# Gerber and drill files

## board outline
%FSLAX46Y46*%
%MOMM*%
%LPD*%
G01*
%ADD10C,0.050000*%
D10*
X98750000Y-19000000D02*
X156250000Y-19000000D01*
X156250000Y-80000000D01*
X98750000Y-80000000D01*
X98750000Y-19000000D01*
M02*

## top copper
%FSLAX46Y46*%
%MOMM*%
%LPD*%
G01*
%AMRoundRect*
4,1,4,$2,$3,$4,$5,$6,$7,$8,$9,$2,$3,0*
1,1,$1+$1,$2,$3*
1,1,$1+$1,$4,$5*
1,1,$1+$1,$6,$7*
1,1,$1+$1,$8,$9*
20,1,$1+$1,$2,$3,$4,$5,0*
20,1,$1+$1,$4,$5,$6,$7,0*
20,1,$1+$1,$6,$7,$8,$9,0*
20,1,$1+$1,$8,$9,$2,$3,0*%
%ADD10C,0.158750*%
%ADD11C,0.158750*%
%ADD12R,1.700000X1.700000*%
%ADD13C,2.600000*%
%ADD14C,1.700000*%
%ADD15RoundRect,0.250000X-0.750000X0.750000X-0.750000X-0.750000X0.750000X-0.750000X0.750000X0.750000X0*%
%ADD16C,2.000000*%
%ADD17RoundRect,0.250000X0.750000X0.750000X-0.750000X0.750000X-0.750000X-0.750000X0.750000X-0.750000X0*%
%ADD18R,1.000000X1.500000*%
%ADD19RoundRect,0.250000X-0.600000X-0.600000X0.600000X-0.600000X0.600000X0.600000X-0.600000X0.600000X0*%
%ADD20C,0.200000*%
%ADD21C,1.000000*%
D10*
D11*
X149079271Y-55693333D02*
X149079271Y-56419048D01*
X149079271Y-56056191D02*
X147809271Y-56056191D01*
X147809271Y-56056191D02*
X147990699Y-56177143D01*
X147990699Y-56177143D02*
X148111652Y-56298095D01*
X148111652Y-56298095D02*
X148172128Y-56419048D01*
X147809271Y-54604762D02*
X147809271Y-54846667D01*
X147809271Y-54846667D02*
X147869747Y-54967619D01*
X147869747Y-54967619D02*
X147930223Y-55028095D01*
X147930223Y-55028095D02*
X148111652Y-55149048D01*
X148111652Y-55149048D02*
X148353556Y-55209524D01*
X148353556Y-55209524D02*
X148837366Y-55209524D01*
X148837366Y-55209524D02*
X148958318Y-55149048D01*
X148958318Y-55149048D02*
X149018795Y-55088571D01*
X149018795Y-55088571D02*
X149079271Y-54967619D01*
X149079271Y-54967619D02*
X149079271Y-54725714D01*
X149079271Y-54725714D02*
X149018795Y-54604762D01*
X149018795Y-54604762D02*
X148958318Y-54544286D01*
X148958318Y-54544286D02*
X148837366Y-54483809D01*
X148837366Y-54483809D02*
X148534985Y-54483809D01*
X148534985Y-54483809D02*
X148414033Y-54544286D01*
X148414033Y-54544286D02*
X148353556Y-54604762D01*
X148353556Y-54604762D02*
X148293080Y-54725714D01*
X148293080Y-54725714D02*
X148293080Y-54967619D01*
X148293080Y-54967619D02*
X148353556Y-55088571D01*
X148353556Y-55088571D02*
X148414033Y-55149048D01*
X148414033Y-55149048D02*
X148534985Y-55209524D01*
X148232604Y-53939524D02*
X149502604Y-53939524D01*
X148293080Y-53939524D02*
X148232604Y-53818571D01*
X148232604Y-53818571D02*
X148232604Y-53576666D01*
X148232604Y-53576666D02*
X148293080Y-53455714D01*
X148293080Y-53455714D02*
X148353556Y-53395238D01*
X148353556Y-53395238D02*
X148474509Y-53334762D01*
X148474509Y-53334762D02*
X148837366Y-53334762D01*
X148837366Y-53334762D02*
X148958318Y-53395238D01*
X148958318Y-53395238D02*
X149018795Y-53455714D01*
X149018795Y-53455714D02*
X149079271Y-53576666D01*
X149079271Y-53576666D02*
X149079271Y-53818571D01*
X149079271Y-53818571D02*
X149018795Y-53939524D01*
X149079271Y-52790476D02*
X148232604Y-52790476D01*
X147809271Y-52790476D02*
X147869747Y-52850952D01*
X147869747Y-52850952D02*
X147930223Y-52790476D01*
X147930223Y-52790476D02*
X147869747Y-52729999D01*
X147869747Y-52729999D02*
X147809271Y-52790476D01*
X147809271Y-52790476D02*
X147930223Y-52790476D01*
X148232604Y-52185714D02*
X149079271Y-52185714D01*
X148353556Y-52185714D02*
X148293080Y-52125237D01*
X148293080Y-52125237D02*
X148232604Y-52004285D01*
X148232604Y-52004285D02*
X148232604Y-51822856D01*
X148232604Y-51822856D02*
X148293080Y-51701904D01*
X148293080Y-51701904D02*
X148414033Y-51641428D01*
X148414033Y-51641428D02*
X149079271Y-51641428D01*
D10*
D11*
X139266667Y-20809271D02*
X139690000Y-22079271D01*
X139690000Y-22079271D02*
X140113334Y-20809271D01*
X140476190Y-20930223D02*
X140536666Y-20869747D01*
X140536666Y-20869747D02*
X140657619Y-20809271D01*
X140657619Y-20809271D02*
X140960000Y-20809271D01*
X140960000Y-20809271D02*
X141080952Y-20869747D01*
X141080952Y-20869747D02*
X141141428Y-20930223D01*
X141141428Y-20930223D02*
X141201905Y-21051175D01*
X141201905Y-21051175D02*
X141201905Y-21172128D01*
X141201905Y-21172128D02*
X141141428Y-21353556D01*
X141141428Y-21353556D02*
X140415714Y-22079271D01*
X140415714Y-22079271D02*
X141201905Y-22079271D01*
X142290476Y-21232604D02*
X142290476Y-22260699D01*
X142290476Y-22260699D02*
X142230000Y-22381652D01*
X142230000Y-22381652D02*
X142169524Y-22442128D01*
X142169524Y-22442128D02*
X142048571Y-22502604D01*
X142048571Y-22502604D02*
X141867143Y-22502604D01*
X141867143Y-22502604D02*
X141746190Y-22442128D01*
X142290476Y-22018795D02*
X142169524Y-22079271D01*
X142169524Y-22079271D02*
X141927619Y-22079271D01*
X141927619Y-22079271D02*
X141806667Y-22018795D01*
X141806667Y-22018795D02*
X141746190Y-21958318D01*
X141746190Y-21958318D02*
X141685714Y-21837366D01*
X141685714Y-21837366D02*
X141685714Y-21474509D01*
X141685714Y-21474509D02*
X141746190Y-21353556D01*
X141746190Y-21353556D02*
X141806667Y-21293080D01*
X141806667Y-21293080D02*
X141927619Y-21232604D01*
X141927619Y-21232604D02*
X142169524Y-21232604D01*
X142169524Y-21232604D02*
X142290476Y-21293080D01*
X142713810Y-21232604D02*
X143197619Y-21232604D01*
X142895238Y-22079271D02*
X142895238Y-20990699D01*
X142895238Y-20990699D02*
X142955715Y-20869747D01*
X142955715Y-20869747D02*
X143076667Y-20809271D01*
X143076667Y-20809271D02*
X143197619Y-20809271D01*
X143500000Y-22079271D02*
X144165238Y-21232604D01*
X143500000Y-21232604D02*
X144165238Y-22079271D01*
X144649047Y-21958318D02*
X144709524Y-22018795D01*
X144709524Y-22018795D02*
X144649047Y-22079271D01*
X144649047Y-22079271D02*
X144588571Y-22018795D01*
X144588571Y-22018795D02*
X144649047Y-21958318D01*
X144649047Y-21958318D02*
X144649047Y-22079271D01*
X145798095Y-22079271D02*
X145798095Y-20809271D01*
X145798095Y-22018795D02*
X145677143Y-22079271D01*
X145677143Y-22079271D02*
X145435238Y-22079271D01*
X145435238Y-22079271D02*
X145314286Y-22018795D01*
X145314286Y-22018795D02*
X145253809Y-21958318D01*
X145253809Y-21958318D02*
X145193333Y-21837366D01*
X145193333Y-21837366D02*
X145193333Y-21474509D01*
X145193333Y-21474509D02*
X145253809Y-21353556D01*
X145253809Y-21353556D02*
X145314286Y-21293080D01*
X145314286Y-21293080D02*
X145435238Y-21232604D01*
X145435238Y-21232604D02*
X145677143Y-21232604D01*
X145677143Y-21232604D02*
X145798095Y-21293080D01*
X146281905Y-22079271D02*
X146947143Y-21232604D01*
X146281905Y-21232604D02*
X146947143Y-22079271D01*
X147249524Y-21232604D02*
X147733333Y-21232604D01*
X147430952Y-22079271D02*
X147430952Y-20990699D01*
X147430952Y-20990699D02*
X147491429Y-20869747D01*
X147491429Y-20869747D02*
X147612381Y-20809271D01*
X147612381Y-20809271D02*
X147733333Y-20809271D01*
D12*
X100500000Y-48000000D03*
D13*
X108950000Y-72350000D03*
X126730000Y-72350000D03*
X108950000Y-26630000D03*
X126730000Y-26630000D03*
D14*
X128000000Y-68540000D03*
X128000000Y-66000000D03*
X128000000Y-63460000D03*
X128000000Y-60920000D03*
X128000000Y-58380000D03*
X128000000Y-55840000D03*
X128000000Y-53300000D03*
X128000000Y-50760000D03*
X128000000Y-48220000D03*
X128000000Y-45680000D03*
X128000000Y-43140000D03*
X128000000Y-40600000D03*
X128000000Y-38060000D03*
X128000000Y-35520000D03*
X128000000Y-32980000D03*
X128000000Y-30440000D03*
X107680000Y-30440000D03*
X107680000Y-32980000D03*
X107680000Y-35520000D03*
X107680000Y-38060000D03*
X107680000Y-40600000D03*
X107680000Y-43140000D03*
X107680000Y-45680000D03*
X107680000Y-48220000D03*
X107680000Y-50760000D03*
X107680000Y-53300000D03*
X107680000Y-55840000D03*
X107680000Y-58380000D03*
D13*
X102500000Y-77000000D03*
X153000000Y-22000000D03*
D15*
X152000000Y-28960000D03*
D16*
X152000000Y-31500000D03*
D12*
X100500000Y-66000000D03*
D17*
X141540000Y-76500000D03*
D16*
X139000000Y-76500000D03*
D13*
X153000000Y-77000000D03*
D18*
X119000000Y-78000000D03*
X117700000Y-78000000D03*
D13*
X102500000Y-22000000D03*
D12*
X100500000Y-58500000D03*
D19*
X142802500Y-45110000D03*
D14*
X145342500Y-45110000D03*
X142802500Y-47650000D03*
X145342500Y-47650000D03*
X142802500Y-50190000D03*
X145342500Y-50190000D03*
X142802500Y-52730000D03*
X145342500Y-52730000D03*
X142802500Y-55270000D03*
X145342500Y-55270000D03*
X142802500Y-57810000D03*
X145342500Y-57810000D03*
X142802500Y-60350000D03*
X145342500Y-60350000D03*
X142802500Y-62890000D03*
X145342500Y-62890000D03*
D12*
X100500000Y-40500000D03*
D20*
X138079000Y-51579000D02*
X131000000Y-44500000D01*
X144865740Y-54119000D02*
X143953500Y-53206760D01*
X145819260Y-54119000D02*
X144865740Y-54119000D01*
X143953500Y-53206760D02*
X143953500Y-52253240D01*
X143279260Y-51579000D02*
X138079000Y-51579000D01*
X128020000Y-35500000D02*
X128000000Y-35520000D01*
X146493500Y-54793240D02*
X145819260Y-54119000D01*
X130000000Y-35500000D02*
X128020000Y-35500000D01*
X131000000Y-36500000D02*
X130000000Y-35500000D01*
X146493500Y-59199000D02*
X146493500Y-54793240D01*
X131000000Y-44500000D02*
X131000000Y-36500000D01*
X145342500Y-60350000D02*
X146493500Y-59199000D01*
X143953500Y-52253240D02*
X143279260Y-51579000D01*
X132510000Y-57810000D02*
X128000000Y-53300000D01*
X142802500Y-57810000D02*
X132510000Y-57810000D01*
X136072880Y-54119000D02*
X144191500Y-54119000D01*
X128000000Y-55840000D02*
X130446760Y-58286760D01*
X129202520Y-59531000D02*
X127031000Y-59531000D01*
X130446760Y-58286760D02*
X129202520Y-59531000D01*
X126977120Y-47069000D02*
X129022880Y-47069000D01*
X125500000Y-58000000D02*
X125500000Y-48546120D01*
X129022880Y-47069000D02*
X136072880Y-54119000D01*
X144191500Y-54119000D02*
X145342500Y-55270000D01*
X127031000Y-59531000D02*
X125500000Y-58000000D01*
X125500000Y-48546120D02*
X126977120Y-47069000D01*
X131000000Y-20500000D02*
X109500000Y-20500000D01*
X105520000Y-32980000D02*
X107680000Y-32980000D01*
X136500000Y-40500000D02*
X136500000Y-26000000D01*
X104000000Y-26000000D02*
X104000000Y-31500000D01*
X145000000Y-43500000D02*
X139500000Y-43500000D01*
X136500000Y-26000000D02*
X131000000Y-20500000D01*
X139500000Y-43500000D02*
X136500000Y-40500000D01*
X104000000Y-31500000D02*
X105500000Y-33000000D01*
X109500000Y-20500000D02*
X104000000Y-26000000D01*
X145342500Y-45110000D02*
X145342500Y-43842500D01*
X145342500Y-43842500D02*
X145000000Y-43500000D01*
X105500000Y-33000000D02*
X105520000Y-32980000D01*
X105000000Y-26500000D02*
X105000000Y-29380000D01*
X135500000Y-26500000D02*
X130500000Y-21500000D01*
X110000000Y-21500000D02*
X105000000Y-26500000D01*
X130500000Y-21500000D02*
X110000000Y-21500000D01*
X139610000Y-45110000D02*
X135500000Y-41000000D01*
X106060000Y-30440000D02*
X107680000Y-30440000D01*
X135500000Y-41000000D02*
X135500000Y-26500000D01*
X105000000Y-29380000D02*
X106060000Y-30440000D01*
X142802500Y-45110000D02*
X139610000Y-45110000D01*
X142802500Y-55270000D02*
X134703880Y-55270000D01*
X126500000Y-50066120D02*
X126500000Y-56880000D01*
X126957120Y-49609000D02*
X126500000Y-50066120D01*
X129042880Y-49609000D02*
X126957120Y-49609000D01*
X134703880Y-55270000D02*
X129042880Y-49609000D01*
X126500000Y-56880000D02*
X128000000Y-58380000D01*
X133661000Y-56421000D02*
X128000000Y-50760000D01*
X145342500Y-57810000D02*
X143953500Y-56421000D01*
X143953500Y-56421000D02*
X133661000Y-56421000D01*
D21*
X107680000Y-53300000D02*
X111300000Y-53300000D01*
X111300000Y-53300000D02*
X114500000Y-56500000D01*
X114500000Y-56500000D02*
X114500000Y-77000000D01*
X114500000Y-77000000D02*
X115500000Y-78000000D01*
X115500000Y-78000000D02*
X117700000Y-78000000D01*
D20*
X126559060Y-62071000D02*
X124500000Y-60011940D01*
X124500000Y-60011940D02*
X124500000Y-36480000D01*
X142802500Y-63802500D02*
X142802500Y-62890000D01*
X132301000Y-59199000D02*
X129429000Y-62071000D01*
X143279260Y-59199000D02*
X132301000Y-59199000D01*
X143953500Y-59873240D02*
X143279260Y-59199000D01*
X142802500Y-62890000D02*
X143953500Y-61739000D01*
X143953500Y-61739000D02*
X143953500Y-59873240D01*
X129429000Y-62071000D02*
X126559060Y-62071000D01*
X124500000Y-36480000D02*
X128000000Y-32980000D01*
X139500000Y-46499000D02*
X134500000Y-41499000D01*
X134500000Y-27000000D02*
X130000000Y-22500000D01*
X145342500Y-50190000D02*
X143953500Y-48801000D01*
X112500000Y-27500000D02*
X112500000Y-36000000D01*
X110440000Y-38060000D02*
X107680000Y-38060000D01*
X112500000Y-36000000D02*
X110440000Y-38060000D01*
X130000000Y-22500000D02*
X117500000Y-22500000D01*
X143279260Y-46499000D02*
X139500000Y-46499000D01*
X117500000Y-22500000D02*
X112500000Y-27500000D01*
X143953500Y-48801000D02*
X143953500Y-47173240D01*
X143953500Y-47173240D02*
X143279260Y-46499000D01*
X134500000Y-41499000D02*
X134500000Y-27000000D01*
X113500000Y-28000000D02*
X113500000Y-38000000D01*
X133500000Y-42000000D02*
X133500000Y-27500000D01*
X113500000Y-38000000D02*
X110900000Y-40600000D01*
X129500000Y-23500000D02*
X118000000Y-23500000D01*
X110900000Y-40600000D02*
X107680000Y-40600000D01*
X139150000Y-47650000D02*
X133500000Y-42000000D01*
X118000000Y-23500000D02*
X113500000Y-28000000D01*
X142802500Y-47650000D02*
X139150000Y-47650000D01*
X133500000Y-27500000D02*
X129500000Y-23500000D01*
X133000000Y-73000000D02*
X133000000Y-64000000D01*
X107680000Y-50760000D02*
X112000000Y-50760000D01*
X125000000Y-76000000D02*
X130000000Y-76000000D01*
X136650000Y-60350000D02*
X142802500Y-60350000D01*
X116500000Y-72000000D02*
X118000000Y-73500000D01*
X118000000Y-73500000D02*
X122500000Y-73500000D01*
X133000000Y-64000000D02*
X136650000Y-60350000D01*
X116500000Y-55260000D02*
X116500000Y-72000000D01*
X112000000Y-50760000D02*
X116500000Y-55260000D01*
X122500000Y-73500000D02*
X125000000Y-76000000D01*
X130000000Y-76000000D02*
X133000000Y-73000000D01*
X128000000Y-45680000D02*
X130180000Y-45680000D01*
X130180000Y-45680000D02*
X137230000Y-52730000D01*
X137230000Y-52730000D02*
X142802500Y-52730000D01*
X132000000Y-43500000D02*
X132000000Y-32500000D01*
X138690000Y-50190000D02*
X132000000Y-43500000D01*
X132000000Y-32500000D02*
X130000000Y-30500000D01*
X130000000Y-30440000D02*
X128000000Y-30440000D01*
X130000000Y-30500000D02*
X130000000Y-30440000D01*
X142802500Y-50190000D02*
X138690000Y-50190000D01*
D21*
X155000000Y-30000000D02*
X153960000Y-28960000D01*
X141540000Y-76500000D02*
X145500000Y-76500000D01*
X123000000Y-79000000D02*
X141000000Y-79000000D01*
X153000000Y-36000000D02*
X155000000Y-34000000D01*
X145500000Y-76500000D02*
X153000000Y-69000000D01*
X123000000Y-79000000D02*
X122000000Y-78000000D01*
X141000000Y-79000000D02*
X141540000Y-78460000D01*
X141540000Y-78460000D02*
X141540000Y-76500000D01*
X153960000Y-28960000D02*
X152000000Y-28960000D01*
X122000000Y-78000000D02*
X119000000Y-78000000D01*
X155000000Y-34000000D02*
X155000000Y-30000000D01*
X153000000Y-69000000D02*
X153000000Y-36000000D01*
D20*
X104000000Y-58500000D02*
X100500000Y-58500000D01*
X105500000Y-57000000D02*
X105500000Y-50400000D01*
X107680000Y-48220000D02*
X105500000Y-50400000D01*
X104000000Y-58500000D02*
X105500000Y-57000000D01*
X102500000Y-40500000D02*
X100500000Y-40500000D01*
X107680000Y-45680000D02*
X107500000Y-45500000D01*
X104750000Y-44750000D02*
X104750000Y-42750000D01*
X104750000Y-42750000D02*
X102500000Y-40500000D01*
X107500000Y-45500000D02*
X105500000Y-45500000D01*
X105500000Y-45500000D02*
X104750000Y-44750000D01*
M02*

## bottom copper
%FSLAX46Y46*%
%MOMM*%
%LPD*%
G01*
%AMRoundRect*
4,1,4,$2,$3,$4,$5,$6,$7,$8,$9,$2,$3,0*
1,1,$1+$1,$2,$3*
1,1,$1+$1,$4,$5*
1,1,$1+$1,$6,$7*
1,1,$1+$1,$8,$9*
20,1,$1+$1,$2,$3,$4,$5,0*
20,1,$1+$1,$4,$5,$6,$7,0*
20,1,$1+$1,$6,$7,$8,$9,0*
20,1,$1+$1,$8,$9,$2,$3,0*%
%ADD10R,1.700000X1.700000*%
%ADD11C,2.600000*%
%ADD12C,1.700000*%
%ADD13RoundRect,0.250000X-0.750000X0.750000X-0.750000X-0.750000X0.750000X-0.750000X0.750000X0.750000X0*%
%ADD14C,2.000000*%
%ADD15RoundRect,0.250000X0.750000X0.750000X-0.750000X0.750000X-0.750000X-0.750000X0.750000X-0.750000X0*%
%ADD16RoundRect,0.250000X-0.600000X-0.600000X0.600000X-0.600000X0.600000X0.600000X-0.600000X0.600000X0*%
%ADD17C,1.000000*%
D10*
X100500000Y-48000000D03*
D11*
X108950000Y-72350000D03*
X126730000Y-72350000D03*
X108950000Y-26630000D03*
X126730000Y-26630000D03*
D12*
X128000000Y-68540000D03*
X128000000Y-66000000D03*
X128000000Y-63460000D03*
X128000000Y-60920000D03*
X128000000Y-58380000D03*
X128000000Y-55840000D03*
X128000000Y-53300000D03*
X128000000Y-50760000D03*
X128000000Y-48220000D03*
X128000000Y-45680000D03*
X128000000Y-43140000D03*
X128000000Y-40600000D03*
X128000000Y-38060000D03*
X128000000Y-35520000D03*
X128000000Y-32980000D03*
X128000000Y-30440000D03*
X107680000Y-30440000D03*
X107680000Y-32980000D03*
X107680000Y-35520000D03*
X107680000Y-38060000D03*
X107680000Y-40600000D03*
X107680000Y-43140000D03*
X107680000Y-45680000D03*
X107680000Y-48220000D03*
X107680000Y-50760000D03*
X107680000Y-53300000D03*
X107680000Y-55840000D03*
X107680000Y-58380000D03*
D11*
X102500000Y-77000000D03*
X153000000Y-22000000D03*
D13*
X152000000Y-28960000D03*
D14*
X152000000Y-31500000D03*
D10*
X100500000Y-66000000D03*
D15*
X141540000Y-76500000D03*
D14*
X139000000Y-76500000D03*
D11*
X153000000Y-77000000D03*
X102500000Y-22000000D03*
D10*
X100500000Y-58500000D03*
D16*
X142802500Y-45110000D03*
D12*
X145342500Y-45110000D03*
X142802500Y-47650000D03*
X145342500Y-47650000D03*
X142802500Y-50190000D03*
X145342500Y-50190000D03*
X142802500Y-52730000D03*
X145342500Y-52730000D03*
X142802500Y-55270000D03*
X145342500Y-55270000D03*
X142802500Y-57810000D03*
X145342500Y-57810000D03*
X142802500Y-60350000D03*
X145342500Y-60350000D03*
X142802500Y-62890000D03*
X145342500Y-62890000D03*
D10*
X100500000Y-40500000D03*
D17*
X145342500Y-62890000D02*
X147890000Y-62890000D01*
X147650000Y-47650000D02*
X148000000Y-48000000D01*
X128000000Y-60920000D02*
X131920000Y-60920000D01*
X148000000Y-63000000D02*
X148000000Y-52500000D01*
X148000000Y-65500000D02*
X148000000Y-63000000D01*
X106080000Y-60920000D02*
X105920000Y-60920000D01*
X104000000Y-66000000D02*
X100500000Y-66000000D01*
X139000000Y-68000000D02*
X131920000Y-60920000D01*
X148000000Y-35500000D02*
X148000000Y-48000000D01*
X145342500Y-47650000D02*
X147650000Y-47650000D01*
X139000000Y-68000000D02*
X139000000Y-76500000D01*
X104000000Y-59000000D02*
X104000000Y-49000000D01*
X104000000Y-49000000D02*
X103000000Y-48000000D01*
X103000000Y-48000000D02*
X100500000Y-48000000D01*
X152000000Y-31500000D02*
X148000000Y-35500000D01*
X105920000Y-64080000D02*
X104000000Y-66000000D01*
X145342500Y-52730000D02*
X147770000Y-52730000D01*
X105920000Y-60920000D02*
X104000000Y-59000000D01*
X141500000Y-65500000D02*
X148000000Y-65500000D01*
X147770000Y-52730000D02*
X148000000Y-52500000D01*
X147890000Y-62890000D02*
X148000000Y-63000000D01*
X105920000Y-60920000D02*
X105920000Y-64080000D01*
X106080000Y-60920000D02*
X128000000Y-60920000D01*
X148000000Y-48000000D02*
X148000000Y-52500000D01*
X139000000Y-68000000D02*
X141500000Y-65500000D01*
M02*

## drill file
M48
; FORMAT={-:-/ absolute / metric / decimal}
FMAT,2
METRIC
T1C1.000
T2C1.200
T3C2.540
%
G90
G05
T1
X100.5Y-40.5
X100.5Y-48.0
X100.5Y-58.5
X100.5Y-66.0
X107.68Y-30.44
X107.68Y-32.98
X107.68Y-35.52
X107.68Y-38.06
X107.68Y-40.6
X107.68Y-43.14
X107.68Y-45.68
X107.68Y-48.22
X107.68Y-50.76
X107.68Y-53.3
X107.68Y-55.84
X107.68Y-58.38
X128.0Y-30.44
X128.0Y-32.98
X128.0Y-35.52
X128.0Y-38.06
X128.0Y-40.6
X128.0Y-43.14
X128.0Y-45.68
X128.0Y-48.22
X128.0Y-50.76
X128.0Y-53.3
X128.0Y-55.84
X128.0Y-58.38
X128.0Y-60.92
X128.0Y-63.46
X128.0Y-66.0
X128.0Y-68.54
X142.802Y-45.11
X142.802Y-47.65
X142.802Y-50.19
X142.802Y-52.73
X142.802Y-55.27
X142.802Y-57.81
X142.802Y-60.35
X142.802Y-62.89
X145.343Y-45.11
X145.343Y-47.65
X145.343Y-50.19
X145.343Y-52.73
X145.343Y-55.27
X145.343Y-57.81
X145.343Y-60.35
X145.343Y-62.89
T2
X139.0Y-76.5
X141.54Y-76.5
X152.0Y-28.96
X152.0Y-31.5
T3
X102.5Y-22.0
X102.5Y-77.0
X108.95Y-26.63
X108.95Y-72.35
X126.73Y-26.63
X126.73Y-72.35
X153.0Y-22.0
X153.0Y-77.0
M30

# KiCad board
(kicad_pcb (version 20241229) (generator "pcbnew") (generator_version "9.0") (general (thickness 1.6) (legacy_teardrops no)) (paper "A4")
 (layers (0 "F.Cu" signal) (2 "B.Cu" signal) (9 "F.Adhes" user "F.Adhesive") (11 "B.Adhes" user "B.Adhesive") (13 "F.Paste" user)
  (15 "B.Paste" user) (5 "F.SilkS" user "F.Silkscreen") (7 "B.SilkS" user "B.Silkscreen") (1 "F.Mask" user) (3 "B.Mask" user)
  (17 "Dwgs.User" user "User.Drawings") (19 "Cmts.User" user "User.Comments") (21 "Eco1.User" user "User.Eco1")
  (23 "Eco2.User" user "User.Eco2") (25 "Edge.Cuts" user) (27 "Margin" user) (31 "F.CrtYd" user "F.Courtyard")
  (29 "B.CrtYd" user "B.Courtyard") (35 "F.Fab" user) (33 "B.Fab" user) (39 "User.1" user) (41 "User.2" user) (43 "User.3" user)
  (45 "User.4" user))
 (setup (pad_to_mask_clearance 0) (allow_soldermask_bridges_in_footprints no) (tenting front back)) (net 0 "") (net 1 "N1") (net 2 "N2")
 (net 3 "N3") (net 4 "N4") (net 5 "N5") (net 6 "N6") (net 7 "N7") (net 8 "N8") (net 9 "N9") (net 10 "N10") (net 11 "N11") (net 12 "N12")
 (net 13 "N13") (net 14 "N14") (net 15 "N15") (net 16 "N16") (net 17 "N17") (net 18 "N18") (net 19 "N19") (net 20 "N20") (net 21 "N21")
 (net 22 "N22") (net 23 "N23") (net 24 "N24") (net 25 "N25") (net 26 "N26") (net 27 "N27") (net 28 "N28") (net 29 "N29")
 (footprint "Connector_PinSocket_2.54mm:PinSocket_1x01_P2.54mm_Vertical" (layer "F.Cu") (at 100.5 48 -90)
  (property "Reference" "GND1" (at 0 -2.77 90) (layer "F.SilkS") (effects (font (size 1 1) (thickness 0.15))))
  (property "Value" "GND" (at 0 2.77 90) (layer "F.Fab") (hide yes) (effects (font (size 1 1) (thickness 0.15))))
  (pad "1" thru_hole rect (at 0 0 270) (size 1.7 1.7) (drill 1) (layers "*.Cu" "*.Mask") (remove_unused_layers no) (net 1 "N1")))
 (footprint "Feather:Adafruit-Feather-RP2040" (layer "F.Cu") (at 117.84 49.49 90)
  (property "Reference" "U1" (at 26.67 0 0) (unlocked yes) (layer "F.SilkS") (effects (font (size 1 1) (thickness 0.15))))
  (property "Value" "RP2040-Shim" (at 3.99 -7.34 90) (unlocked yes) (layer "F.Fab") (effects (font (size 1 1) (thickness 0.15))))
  (pad "" np_thru_hole circle (at -22.86 -8.89 90) (size 2.6 2.6) (drill 2.54) (layers "*.Cu" "*.Mask") (solder_mask_margin 1.3)
   (clearance 1.3))
  (pad "" np_thru_hole circle (at -22.86 8.89 90) (size 2.6 2.6) (drill 2.54) (layers "*.Cu" "*.Mask") (solder_mask_margin 1.3)
   (clearance 1.3))
  (pad "" np_thru_hole circle (at 22.86 -8.89 90) (size 2.6 2.6) (drill 2.54) (layers "*.Cu" "*.Mask") (solder_mask_margin 1.3)
   (clearance 1.3))
  (pad "" np_thru_hole circle (at 22.86 8.89 90) (size 2.6 2.6) (drill 2.54) (layers "*.Cu" "*.Mask") (solder_mask_margin 1.3)
   (clearance 1.3))
  (pad "1" thru_hole circle (at -19.05 10.16 90) (size 1.7 1.7) (drill 1) (layers "*.Cu" "*.Mask") (remove_unused_layers no) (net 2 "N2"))
  (pad "2" thru_hole circle (at -16.51 10.16 90) (size 1.7 1.7) (drill 1) (layers "*.Cu" "*.Mask") (remove_unused_layers no) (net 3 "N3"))
  (pad "3" thru_hole circle (at -13.97 10.16 90) (size 1.7 1.7) (drill 1) (layers "*.Cu" "*.Mask") (remove_unused_layers no) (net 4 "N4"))
  (pad "4" thru_hole circle (at -11.43 10.16 90) (size 1.7 1.7) (drill 1) (layers "*.Cu" "*.Mask") (remove_unused_layers no) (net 1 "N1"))
  (pad "5" thru_hole circle (at -8.89 10.16 90) (size 1.7 1.7) (drill 1) (layers "*.Cu" "*.Mask") (remove_unused_layers no) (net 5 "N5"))
  (pad "6" thru_hole circle (at -6.35 10.16 90) (size 1.7 1.7) (drill 1) (layers "*.Cu" "*.Mask") (remove_unused_layers no) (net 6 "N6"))
  (pad "7" thru_hole circle (at -3.81 10.16 90) (size 1.7 1.7) (drill 1) (layers "*.Cu" "*.Mask") (remove_unused_layers no) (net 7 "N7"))
  (pad "8" thru_hole circle (at -1.27 10.16 90) (size 1.7 1.7) (drill 1) (layers "*.Cu" "*.Mask") (remove_unused_layers no) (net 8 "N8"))
  (pad "9" thru_hole circle (at 1.27 10.16 90) (size 1.7 1.7) (drill 1) (layers "*.Cu" "*.Mask") (remove_unused_layers no) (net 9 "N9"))
  (pad "10" thru_hole circle (at 3.81 10.16 90) (size 1.7 1.7) (drill 1) (layers "*.Cu" "*.Mask") (remove_unused_layers no) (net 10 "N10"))
  (pad "11" thru_hole circle (at 6.35 10.16 90) (size 1.7 1.7) (drill 1) (layers "*.Cu" "*.Mask") (remove_unused_layers no) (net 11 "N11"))
  (pad "12" thru_hole circle (at 8.89 10.16 90) (size 1.7 1.7) (drill 1) (layers "*.Cu" "*.Mask") (remove_unused_layers no) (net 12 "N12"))
  (pad "13" thru_hole circle (at 11.43 10.16 90) (size 1.7 1.7) (drill 1) (layers "*.Cu" "*.Mask") (remove_unused_layers no) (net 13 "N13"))
  (pad "14" thru_hole circle (at 13.97 10.16 90) (size 1.7 1.7) (drill 1) (layers "*.Cu" "*.Mask") (remove_unused_layers no) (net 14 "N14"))
  (pad "15" thru_hole circle (at 16.51 10.16 90) (size 1.7 1.7) (drill 1) (layers "*.Cu" "*.Mask") (remove_unused_layers no) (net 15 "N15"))
  (pad "16" thru_hole circle (at 19.05 10.16 90) (size 1.7 1.7) (drill 1) (layers "*.Cu" "*.Mask") (remove_unused_layers no) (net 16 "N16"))
  (pad "17" thru_hole circle (at 19.05 -10.16 90) (size 1.7 1.7) (drill 1) (layers "*.Cu" "*.Mask") (remove_unused_layers no) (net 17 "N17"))
  (pad "18" thru_hole circle (at 16.51 -10.16 90) (size 1.7 1.7) (drill 1) (layers "*.Cu" "*.Mask") (remove_unused_layers no) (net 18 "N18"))
  (pad "19" thru_hole circle (at 13.97 -10.16 90) (size 1.7 1.7) (drill 1) (layers "*.Cu" "*.Mask") (remove_unused_layers no) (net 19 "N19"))
  (pad "20" thru_hole circle (at 11.43 -10.16 90) (size 1.7 1.7) (drill 1) (layers "*.Cu" "*.Mask") (remove_unused_layers no) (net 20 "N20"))
  (pad "21" thru_hole circle (at 8.89 -10.16 90) (size 1.7 1.7) (drill 1) (layers "*.Cu" "*.Mask") (remove_unused_layers no) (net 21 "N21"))
  (pad "22" thru_hole circle (at 6.35 -10.16 90) (size 1.7 1.7) (drill 1) (layers "*.Cu" "*.Mask") (remove_unused_layers no) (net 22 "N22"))
  (pad "23" thru_hole circle (at 3.81 -10.16 90) (size 1.7 1.7) (drill 1) (layers "*.Cu" "*.Mask") (remove_unused_layers no) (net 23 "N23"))
  (pad "24" thru_hole circle (at 1.27 -10.16 90) (size 1.7 1.7) (drill 1) (layers "*.Cu" "*.Mask") (remove_unused_layers no) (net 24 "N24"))
  (pad "25" thru_hole circle (at -1.27 -10.16 90) (size 1.7 1.7) (drill 1) (layers "*.Cu" "*.Mask") (remove_unused_layers no) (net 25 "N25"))
  (pad "26" thru_hole circle (at -3.81 -10.16 90) (size 1.7 1.7) (drill 1) (layers "*.Cu" "*.Mask") (remove_unused_layers no) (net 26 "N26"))
  (pad "27" thru_hole circle (at -6.35 -10.16 90) (size 1.7 1.7) (drill 1) (layers "*.Cu" "*.Mask") (remove_unused_layers no) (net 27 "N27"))
  (pad "28" thru_hole circle (at -8.89 -10.16 90) (size 1.7 1.7) (drill 1) (layers "*.Cu" "*.Mask") (remove_unused_layers no) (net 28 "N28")))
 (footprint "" (layer "F.Cu") (at 102.5 77)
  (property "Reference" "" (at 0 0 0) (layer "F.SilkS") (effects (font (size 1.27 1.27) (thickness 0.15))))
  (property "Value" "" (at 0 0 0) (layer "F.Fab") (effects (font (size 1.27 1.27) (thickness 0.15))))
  (pad "" np_thru_hole circle (at 0 0 90) (size 2.6 2.6) (drill 2.54) (layers "*.Cu" "*.Mask") (solder_mask_margin 1.3) (clearance 1.3)))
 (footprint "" (layer "F.Cu") (at 153 22)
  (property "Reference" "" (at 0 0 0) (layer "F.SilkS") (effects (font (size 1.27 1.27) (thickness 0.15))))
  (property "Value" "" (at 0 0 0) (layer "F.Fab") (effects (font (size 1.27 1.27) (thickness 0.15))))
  (pad "" np_thru_hole circle (at 0 0 90) (size 2.6 2.6) (drill 2.54) (layers "*.Cu" "*.Mask") (solder_mask_margin 1.3) (clearance 1.3)))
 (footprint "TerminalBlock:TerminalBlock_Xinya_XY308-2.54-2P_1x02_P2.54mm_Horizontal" (layer "F.Cu") (at 152 28.96 -90)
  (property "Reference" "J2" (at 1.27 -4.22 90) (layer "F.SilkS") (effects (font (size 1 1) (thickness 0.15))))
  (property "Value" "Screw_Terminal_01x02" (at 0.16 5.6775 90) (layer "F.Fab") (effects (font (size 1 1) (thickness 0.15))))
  (pad "1" thru_hole roundrect (at 0 0 270) (size 2 2) (drill 1.2) (layers "*.Cu" "*.Mask") (remove_unused_layers no)
   (roundrect_rratio 0.125) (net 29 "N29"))
  (pad "2" thru_hole circle (at 2.54 0 270) (size 2 2) (drill 1.2) (layers "*.Cu" "*.Mask") (remove_unused_layers no) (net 1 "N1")))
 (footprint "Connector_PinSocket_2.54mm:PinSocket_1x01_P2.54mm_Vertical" (layer "F.Cu") (at 100.5 66 -90)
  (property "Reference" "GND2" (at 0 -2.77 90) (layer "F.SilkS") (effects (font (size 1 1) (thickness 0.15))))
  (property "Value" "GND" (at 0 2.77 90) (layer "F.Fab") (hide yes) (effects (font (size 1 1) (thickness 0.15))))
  (pad "1" thru_hole rect (at 0 0 270) (size 1.7 1.7) (drill 1) (layers "*.Cu" "*.Mask") (remove_unused_layers no) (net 1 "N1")))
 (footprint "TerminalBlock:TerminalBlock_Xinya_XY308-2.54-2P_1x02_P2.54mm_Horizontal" (layer "F.Cu") (at 141.54 76.5 180)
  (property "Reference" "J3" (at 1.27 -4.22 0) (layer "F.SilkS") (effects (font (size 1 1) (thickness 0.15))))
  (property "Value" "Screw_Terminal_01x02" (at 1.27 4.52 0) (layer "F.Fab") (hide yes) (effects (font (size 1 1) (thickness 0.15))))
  (pad "1" thru_hole roundrect (at 0 0 180) (size 2 2) (drill 1.2) (layers "*.Cu" "*.Mask") (remove_unused_layers no)
   (roundrect_rratio 0.125) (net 29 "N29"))
  (pad "2" thru_hole circle (at 2.54 0 180) (size 2 2) (drill 1.2) (layers "*.Cu" "*.Mask") (remove_unused_layers no) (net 1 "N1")))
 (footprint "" (layer "F.Cu") (at 153 77)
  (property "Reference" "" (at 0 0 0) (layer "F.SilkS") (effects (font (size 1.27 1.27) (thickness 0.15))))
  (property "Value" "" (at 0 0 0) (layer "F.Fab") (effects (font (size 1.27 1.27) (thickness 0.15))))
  (pad "" np_thru_hole circle (at 0 0 90) (size 2.6 2.6) (drill 2.54) (layers "*.Cu" "*.Mask") (solder_mask_margin 1.3) (clearance 1.3)))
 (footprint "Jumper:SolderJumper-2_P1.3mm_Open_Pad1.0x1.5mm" (layer "F.Cu") (at 118.35 78 180)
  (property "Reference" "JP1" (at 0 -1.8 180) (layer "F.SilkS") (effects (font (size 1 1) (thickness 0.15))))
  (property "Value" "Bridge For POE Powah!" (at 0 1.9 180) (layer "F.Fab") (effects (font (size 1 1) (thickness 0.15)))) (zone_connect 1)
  (pad "1" smd rect (at -0.65 0 180) (size 1 1.5) (layers "F.Cu" "F.Mask") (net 29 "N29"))
  (pad "2" smd rect (at 0.65 0 180) (size 1 1.5) (layers "F.Cu" "F.Mask") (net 26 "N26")))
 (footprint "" (layer "F.Cu") (at 102.5 22)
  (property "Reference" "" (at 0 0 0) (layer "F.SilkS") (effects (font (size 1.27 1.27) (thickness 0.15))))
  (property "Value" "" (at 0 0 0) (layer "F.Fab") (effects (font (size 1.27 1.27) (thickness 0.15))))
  (pad "" np_thru_hole circle (at 0 0 90) (size 2.6 2.6) (drill 2.54) (layers "*.Cu" "*.Mask") (solder_mask_margin 1.3) (clearance 1.3)))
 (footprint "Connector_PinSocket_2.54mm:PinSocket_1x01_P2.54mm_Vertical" (layer "F.Cu") (at 100.5 58.5 -90)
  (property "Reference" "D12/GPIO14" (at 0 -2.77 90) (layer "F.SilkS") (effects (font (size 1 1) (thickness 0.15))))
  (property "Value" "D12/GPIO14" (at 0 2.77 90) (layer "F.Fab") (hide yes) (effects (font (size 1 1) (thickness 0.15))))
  (pad "1" thru_hole rect (at 0 0 270) (size 1.7 1.7) (drill 1) (layers "*.Cu" "*.Mask") (remove_unused_layers no) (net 24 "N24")))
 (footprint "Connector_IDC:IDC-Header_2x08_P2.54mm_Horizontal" (layer "F.Cu") (at 142.8025 45.11)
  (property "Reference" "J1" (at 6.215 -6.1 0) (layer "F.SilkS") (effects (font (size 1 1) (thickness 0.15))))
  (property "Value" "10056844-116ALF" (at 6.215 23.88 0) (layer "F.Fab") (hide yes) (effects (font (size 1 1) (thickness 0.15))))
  (pad "1" thru_hole roundrect (at 0 0) (size 1.7 1.7) (drill 1) (layers "*.Cu" "*.Mask") (remove_unused_layers no)
   (roundrect_rratio 0.147059) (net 17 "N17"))
  (pad "2" thru_hole circle (at 2.54 0) (size 1.7 1.7) (drill 1) (layers "*.Cu" "*.Mask") (remove_unused_layers no) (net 18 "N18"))
  (pad "3" thru_hole circle (at 0 2.54) (size 1.7 1.7) (drill 1) (layers "*.Cu" "*.Mask") (remove_unused_layers no) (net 21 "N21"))
  (pad "4" thru_hole circle (at 2.54 2.54) (size 1.7 1.7) (drill 1) (layers "*.Cu" "*.Mask") (remove_unused_layers no) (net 1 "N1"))
  (pad "5" thru_hole circle (at 0 5.08) (size 1.7 1.7) (drill 1) (layers "*.Cu" "*.Mask") (remove_unused_layers no) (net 16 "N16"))
  (pad "6" thru_hole circle (at 2.54 5.08) (size 1.7 1.7) (drill 1) (layers "*.Cu" "*.Mask") (remove_unused_layers no) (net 20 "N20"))
  (pad "7" thru_hole circle (at 0 7.62) (size 1.7 1.7) (drill 1) (layers "*.Cu" "*.Mask") (remove_unused_layers no) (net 10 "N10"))
  (pad "8" thru_hole circle (at 2.54 7.62) (size 1.7 1.7) (drill 1) (layers "*.Cu" "*.Mask") (remove_unused_layers no) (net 1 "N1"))
  (pad "9" thru_hole circle (at 0 10.16) (size 1.7 1.7) (drill 1) (layers "*.Cu" "*.Mask") (remove_unused_layers no) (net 5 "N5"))
  (pad "10" thru_hole circle (at 2.54 10.16) (size 1.7 1.7) (drill 1) (layers "*.Cu" "*.Mask") (remove_unused_layers no) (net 6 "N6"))
  (pad "11" thru_hole circle (at 0 12.7) (size 1.7 1.7) (drill 1) (layers "*.Cu" "*.Mask") (remove_unused_layers no) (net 7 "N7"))
  (pad "12" thru_hole circle (at 2.54 12.7) (size 1.7 1.7) (drill 1) (layers "*.Cu" "*.Mask") (remove_unused_layers no) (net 8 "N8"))
  (pad "13" thru_hole circle (at 0 15.24) (size 1.7 1.7) (drill 1) (layers "*.Cu" "*.Mask") (remove_unused_layers no) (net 25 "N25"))
  (pad "14" thru_hole circle (at 2.54 15.24) (size 1.7 1.7) (drill 1) (layers "*.Cu" "*.Mask") (remove_unused_layers no) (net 14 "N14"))
  (pad "15" thru_hole circle (at 0 17.78) (size 1.7 1.7) (drill 1) (layers "*.Cu" "*.Mask") (remove_unused_layers no) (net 15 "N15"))
  (pad "16" thru_hole circle (at 2.54 17.78) (size 1.7 1.7) (drill 1) (layers "*.Cu" "*.Mask") (remove_unused_layers no) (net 1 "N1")))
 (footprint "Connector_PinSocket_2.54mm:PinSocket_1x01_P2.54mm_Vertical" (layer "F.Cu") (at 100.5 40.5 -90)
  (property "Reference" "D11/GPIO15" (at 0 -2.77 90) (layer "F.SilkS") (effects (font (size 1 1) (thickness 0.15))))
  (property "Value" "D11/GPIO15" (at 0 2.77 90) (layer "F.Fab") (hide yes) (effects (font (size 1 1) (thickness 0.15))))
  (pad "1" thru_hole rect (at 0 0 270) (size 1.7 1.7) (drill 1) (layers "*.Cu" "*.Mask") (remove_unused_layers no) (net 23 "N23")))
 (gr_rect (start 98.75 19) (end 156.25 80) (stroke (width 0.05) (type solid)) (fill no) (layer "Edge.Cuts"))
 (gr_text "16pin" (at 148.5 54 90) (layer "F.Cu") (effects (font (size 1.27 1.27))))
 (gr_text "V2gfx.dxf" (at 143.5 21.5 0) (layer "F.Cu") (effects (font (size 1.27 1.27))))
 (segment (start 138.079 51.579) (end 131 44.5) (width 0.2) (layer "F.Cu") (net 14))
 (segment (start 144.86574 54.119) (end 143.9535 53.20676) (width 0.2) (layer "F.Cu") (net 14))
 (segment (start 145.81926 54.119) (end 144.86574 54.119) (width 0.2) (layer "F.Cu") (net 14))
 (segment (start 143.9535 53.20676) (end 143.9535 52.25324) (width 0.2) (layer "F.Cu") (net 14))
 (segment (start 143.27926 51.579) (end 138.079 51.579) (width 0.2) (layer "F.Cu") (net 14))
 (segment (start 128.02 35.5) (end 128 35.52) (width 0.2) (layer "F.Cu") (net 14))
 (segment (start 146.4935 54.79324) (end 145.81926 54.119) (width 0.2) (layer "F.Cu") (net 14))
 (segment (start 130 35.5) (end 128.02 35.5) (width 0.2) (layer "F.Cu") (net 14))
 (segment (start 131 36.5) (end 130 35.5) (width 0.2) (layer "F.Cu") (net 14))
 (segment (start 146.4935 59.199) (end 146.4935 54.79324) (width 0.2) (layer "F.Cu") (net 14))
 (segment (start 131 44.5) (end 131 36.5) (width 0.2) (layer "F.Cu") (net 14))
 (segment (start 145.3425 60.35) (end 146.4935 59.199) (width 0.2) (layer "F.Cu") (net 14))
 (segment (start 143.9535 52.25324) (end 143.27926 51.579) (width 0.2) (layer "F.Cu") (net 14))
 (segment (start 132.51 57.81) (end 128 53.3) (width 0.2) (layer "F.Cu") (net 7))
 (segment (start 142.8025 57.81) (end 132.51 57.81) (width 0.2) (layer "F.Cu") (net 7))
 (segment (start 136.07288 54.119) (end 144.1915 54.119) (width 0.2) (layer "F.Cu") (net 6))
 (segment (start 128 55.84) (end 130.44676 58.28676) (width 0.2) (layer "F.Cu") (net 6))
 (segment (start 129.20252 59.531) (end 127.031 59.531) (width 0.2) (layer "F.Cu") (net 6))
 (segment (start 130.44676 58.28676) (end 129.20252 59.531) (width 0.2) (layer "F.Cu") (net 6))
 (segment (start 126.97712 47.069) (end 129.02288 47.069) (width 0.2) (layer "F.Cu") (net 6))
 (segment (start 125.5 58) (end 125.5 48.54612) (width 0.2) (layer "F.Cu") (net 6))
 (segment (start 129.02288 47.069) (end 136.07288 54.119) (width 0.2) (layer "F.Cu") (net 6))
 (segment (start 144.1915 54.119) (end 145.3425 55.27) (width 0.2) (layer "F.Cu") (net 6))
 (segment (start 127.031 59.531) (end 125.5 58) (width 0.2) (layer "F.Cu") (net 6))
 (segment (start 125.5 48.54612) (end 126.97712 47.069) (width 0.2) (layer "F.Cu") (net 6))
 (segment (start 131 20.5) (end 109.5 20.5) (width 0.2) (layer "F.Cu") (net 18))
 (segment (start 105.52 32.98) (end 107.68 32.98) (width 0.2) (layer "F.Cu") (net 18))
 (segment (start 136.5 40.5) (end 136.5 26) (width 0.2) (layer "F.Cu") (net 18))
 (segment (start 104 26) (end 104 31.5) (width 0.2) (layer "F.Cu") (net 18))
 (segment (start 145 43.5) (end 139.5 43.5) (width 0.2) (layer "F.Cu") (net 18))
 (segment (start 136.5 26) (end 131 20.5) (width 0.2) (layer "F.Cu") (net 18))
 (segment (start 139.5 43.5) (end 136.5 40.5) (width 0.2) (layer "F.Cu") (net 18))
 (segment (start 104 31.5) (end 105.5 33) (width 0.2) (layer "F.Cu") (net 18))
 (segment (start 109.5 20.5) (end 104 26) (width 0.2) (layer "F.Cu") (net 18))
 (segment (start 145.3425 45.11) (end 145.3425 43.8425) (width 0.2) (layer "F.Cu") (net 18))
 (segment (start 145.3425 43.8425) (end 145 43.5) (width 0.2) (layer "F.Cu") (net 18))
 (segment (start 105.5 33) (end 105.52 32.98) (width 0.2) (layer "F.Cu") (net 18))
 (segment (start 105 26.5) (end 105 29.38) (width 0.2) (layer "F.Cu") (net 17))
 (segment (start 135.5 26.5) (end 130.5 21.5) (width 0.2) (layer "F.Cu") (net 17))
 (segment (start 110 21.5) (end 105 26.5) (width 0.2) (layer "F.Cu") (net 17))
 (segment (start 130.5 21.5) (end 110 21.5) (width 0.2) (layer "F.Cu") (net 17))
 (segment (start 139.61 45.11) (end 135.5 41) (width 0.2) (layer "F.Cu") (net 17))
 (segment (start 106.06 30.44) (end 107.68 30.44) (width 0.2) (layer "F.Cu") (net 17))
 (segment (start 135.5 41) (end 135.5 26.5) (width 0.2) (layer "F.Cu") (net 17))
 (segment (start 105 29.38) (end 106.06 30.44) (width 0.2) (layer "F.Cu") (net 17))
 (segment (start 142.8025 45.11) (end 139.61 45.11) (width 0.2) (layer "F.Cu") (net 17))
 (segment (start 142.8025 55.27) (end 134.70388 55.27) (width 0.2) (layer "F.Cu") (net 5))
 (segment (start 126.5 50.06612) (end 126.5 56.88) (width 0.2) (layer "F.Cu") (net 5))
 (segment (start 126.95712 49.609) (end 126.5 50.06612) (width 0.2) (layer "F.Cu") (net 5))
 (segment (start 129.04288 49.609) (end 126.95712 49.609) (width 0.2) (layer "F.Cu") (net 5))
 (segment (start 134.70388 55.27) (end 129.04288 49.609) (width 0.2) (layer "F.Cu") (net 5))
 (segment (start 126.5 56.88) (end 128 58.38) (width 0.2) (layer "F.Cu") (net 5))
 (segment (start 133.661 56.421) (end 128 50.76) (width 0.2) (layer "F.Cu") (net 8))
 (segment (start 145.3425 57.81) (end 143.9535 56.421) (width 0.2) (layer "F.Cu") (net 8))
 (segment (start 143.9535 56.421) (end 133.661 56.421) (width 0.2) (layer "F.Cu") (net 8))
 (segment (start 145.3425 62.89) (end 147.89 62.89) (width 1) (layer "B.Cu") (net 1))
 (segment (start 147.65 47.65) (end 148 48) (width 1) (layer "B.Cu") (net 1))
 (segment (start 128 60.92) (end 131.92 60.92) (width 1) (layer "B.Cu") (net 1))
 (segment (start 148 63) (end 148 52.5) (width 1) (layer "B.Cu") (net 1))
 (segment (start 148 65.5) (end 148 63) (width 1) (layer "B.Cu") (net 1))
 (segment (start 106.08 60.92) (end 105.92 60.92) (width 1) (layer "B.Cu") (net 1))
 (segment (start 104 66) (end 100.5 66) (width 1) (layer "B.Cu") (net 1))
 (segment (start 139 68) (end 131.92 60.92) (width 1) (layer "B.Cu") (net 1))
 (segment (start 148 35.5) (end 148 48) (width 1) (layer "B.Cu") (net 1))
 (segment (start 145.3425 47.65) (end 147.65 47.65) (width 1) (layer "B.Cu") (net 1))
 (segment (start 139 68) (end 139 76.5) (width 1) (layer "B.Cu") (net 1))
 (segment (start 104 59) (end 104 49) (width 1) (layer "B.Cu") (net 1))
 (segment (start 104 49) (end 103 48) (width 1) (layer "B.Cu") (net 1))
 (segment (start 103 48) (end 100.5 48) (width 1) (layer "B.Cu") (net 1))
 (segment (start 152 31.5) (end 148 35.5) (width 1) (layer "B.Cu") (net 1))
 (segment (start 105.92 64.08) (end 104 66) (width 1) (layer "B.Cu") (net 1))
 (segment (start 145.3425 52.73) (end 147.77 52.73) (width 1) (layer "B.Cu") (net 1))
 (segment (start 105.92 60.92) (end 104 59) (width 1) (layer "B.Cu") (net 1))
 (segment (start 141.5 65.5) (end 148 65.5) (width 1) (layer "B.Cu") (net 1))
 (segment (start 147.77 52.73) (end 148 52.5) (width 1) (layer "B.Cu") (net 1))
 (segment (start 147.89 62.89) (end 148 63) (width 1) (layer "B.Cu") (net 1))
 (segment (start 105.92 60.92) (end 105.92 64.08) (width 1) (layer "B.Cu") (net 1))
 (segment (start 106.08 60.92) (end 128 60.92) (width 1) (layer "B.Cu") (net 1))
 (segment (start 148 48) (end 148 52.5) (width 1) (layer "B.Cu") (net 1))
 (segment (start 139 68) (end 141.5 65.5) (width 1) (layer "B.Cu") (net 1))
 (segment (start 107.68 53.3) (end 111.3 53.3) (width 1) (layer "F.Cu") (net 26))
 (segment (start 111.3 53.3) (end 114.5 56.5) (width 1) (layer "F.Cu") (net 26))
 (segment (start 114.5 56.5) (end 114.5 77) (width 1) (layer "F.Cu") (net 26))
 (segment (start 114.5 77) (end 115.5 78) (width 1) (layer "F.Cu") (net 26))
 (segment (start 115.5 78) (end 117.7 78) (width 1) (layer "F.Cu") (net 26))
 (segment (start 126.55906 62.071) (end 124.5 60.01194) (width 0.2) (layer "F.Cu") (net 15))
 (segment (start 124.5 60.01194) (end 124.5 36.48) (width 0.2) (layer "F.Cu") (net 15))
 (segment (start 142.8025 63.8025) (end 142.8025 62.89) (width 0.2) (layer "F.Cu") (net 15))
 (segment (start 132.301 59.199) (end 129.429 62.071) (width 0.2) (layer "F.Cu") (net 15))
 (segment (start 143.27926 59.199) (end 132.301 59.199) (width 0.2) (layer "F.Cu") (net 15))
 (segment (start 143.9535 59.87324) (end 143.27926 59.199) (width 0.2) (layer "F.Cu") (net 15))
 (segment (start 142.8025 62.89) (end 143.9535 61.739) (width 0.2) (layer "F.Cu") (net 15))
 (segment (start 143.9535 61.739) (end 143.9535 59.87324) (width 0.2) (layer "F.Cu") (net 15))
 (segment (start 129.429 62.071) (end 126.55906 62.071) (width 0.2) (layer "F.Cu") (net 15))
 (segment (start 124.5 36.48) (end 128 32.98) (width 0.2) (layer "F.Cu") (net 15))
 (segment (start 139.5 46.499) (end 134.5 41.499) (width 0.2) (layer "F.Cu") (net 20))
 (segment (start 134.5 27) (end 130 22.5) (width 0.2) (layer "F.Cu") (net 20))
 (segment (start 145.3425 50.19) (end 143.9535 48.801) (width 0.2) (layer "F.Cu") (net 20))
 (segment (start 112.5 27.5) (end 112.5 36) (width 0.2) (layer "F.Cu") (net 20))
 (segment (start 110.44 38.06) (end 107.68 38.06) (width 0.2) (layer "F.Cu") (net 20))
 (segment (start 112.5 36) (end 110.44 38.06) (width 0.2) (layer "F.Cu") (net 20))
 (segment (start 130 22.5) (end 117.5 22.5) (width 0.2) (layer "F.Cu") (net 20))
 (segment (start 143.27926 46.499) (end 139.5 46.499) (width 0.2) (layer "F.Cu") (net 20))
 (segment (start 117.5 22.5) (end 112.5 27.5) (width 0.2) (layer "F.Cu") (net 20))
 (segment (start 143.9535 48.801) (end 143.9535 47.17324) (width 0.2) (layer "F.Cu") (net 20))
 (segment (start 143.9535 47.17324) (end 143.27926 46.499) (width 0.2) (layer "F.Cu") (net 20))
 (segment (start 134.5 41.499) (end 134.5 27) (width 0.2) (layer "F.Cu") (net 20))
 (segment (start 113.5 28) (end 113.5 38) (width 0.2) (layer "F.Cu") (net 21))
 (segment (start 133.5 42) (end 133.5 27.5) (width 0.2) (layer "F.Cu") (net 21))
 (segment (start 113.5 38) (end 110.9 40.6) (width 0.2) (layer "F.Cu") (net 21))
 (segment (start 129.5 23.5) (end 118 23.5) (width 0.2) (layer "F.Cu") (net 21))
 (segment (start 110.9 40.6) (end 107.68 40.6) (width 0.2) (layer "F.Cu") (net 21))
 (segment (start 139.15 47.65) (end 133.5 42) (width 0.2) (layer "F.Cu") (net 21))
 (segment (start 118 23.5) (end 113.5 28) (width 0.2) (layer "F.Cu") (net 21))
 (segment (start 142.8025 47.65) (end 139.15 47.65) (width 0.2) (layer "F.Cu") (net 21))
 (segment (start 133.5 27.5) (end 129.5 23.5) (width 0.2) (layer "F.Cu") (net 21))
 (segment (start 133 73) (end 133 64) (width 0.2) (layer "F.Cu") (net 25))
 (segment (start 107.68 50.76) (end 112 50.76) (width 0.2) (layer "F.Cu") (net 25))
 (segment (start 125 76) (end 130 76) (width 0.2) (layer "F.Cu") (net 25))
 (segment (start 136.65 60.35) (end 142.8025 60.35) (width 0.2) (layer "F.Cu") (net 25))
 (segment (start 116.5 72) (end 118 73.5) (width 0.2) (layer "F.Cu") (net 25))
 (segment (start 118 73.5) (end 122.5 73.5) (width 0.2) (layer "F.Cu") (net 25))
 (segment (start 133 64) (end 136.65 60.35) (width 0.2) (layer "F.Cu") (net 25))
 (segment (start 116.5 55.26) (end 116.5 72) (width 0.2) (layer "F.Cu") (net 25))
 (segment (start 112 50.76) (end 116.5 55.26) (width 0.2) (layer "F.Cu") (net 25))
 (segment (start 122.5 73.5) (end 125 76) (width 0.2) (layer "F.Cu") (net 25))
 (segment (start 130 76) (end 133 73) (width 0.2) (layer "F.Cu") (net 25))
 (segment (start 128 45.68) (end 130.18 45.68) (width 0.2) (layer "F.Cu") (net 10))
 (segment (start 130.18 45.68) (end 137.23 52.73) (width 0.2) (layer "F.Cu") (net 10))
 (segment (start 137.23 52.73) (end 142.8025 52.73) (width 0.2) (layer "F.Cu") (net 10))
 (segment (start 132 43.5) (end 132 32.5) (width 0.2) (layer "F.Cu") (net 16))
 (segment (start 138.69 50.19) (end 132 43.5) (width 0.2) (layer "F.Cu") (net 16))
 (segment (start 132 32.5) (end 130 30.5) (width 0.2) (layer "F.Cu") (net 16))
 (segment (start 130 30.44) (end 128 30.44) (width 0.2) (layer "F.Cu") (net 16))
 (segment (start 130 30.5) (end 130 30.44) (width 0.2) (layer "F.Cu") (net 16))
 (segment (start 142.8025 50.19) (end 138.69 50.19) (width 0.2) (layer "F.Cu") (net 16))
 (segment (start 155 30) (end 153.96 28.96) (width 1) (layer "F.Cu") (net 29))
 (segment (start 141.54 76.5) (end 145.5 76.5) (width 1) (layer "F.Cu") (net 29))
 (segment (start 123 79) (end 141 79) (width 1) (layer "F.Cu") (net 29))
 (segment (start 153 36) (end 155 34) (width 1) (layer "F.Cu") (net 29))
 (segment (start 145.5 76.5) (end 153 69) (width 1) (layer "F.Cu") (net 29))
 (segment (start 123 79) (end 122 78) (width 1) (layer "F.Cu") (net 29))
 (segment (start 141 79) (end 141.54 78.46) (width 1) (layer "F.Cu") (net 29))
 (segment (start 141.54 78.46) (end 141.54 76.5) (width 1) (layer "F.Cu") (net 29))
 (segment (start 153.96 28.96) (end 152 28.96) (width 1) (layer "F.Cu") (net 29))
 (segment (start 122 78) (end 119 78) (width 1) (layer "F.Cu") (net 29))
 (segment (start 155 34) (end 155 30) (width 1) (layer "F.Cu") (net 29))
 (segment (start 153 69) (end 153 36) (width 1) (layer "F.Cu") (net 29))
 (segment (start 104 58.5) (end 100.5 58.5) (width 0.2) (layer "F.Cu") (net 24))
 (segment (start 105.5 57) (end 105.5 50.4) (width 0.2) (layer "F.Cu") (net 24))
 (segment (start 107.68 48.22) (end 105.5 50.4) (width 0.2) (layer "F.Cu") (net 24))
 (segment (start 104 58.5) (end 105.5 57) (width 0.2) (layer "F.Cu") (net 24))
 (segment (start 102.5 40.5) (end 100.5 40.5) (width 0.2) (layer "F.Cu") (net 23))
 (segment (start 107.68 45.68) (end 107.5 45.5) (width 0.2) (layer "F.Cu") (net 23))
 (segment (start 104.75 44.75) (end 104.75 42.75) (width 0.2) (layer "F.Cu") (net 23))
 (segment (start 104.75 42.75) (end 102.5 40.5) (width 0.2) (layer "F.Cu") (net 23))
 (segment (start 107.5 45.5) (end 105.5 45.5) (width 0.2) (layer "F.Cu") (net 23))
 (segment (start 105.5 45.5) (end 104.75 44.75) (width 0.2) (layer "F.Cu") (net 23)))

